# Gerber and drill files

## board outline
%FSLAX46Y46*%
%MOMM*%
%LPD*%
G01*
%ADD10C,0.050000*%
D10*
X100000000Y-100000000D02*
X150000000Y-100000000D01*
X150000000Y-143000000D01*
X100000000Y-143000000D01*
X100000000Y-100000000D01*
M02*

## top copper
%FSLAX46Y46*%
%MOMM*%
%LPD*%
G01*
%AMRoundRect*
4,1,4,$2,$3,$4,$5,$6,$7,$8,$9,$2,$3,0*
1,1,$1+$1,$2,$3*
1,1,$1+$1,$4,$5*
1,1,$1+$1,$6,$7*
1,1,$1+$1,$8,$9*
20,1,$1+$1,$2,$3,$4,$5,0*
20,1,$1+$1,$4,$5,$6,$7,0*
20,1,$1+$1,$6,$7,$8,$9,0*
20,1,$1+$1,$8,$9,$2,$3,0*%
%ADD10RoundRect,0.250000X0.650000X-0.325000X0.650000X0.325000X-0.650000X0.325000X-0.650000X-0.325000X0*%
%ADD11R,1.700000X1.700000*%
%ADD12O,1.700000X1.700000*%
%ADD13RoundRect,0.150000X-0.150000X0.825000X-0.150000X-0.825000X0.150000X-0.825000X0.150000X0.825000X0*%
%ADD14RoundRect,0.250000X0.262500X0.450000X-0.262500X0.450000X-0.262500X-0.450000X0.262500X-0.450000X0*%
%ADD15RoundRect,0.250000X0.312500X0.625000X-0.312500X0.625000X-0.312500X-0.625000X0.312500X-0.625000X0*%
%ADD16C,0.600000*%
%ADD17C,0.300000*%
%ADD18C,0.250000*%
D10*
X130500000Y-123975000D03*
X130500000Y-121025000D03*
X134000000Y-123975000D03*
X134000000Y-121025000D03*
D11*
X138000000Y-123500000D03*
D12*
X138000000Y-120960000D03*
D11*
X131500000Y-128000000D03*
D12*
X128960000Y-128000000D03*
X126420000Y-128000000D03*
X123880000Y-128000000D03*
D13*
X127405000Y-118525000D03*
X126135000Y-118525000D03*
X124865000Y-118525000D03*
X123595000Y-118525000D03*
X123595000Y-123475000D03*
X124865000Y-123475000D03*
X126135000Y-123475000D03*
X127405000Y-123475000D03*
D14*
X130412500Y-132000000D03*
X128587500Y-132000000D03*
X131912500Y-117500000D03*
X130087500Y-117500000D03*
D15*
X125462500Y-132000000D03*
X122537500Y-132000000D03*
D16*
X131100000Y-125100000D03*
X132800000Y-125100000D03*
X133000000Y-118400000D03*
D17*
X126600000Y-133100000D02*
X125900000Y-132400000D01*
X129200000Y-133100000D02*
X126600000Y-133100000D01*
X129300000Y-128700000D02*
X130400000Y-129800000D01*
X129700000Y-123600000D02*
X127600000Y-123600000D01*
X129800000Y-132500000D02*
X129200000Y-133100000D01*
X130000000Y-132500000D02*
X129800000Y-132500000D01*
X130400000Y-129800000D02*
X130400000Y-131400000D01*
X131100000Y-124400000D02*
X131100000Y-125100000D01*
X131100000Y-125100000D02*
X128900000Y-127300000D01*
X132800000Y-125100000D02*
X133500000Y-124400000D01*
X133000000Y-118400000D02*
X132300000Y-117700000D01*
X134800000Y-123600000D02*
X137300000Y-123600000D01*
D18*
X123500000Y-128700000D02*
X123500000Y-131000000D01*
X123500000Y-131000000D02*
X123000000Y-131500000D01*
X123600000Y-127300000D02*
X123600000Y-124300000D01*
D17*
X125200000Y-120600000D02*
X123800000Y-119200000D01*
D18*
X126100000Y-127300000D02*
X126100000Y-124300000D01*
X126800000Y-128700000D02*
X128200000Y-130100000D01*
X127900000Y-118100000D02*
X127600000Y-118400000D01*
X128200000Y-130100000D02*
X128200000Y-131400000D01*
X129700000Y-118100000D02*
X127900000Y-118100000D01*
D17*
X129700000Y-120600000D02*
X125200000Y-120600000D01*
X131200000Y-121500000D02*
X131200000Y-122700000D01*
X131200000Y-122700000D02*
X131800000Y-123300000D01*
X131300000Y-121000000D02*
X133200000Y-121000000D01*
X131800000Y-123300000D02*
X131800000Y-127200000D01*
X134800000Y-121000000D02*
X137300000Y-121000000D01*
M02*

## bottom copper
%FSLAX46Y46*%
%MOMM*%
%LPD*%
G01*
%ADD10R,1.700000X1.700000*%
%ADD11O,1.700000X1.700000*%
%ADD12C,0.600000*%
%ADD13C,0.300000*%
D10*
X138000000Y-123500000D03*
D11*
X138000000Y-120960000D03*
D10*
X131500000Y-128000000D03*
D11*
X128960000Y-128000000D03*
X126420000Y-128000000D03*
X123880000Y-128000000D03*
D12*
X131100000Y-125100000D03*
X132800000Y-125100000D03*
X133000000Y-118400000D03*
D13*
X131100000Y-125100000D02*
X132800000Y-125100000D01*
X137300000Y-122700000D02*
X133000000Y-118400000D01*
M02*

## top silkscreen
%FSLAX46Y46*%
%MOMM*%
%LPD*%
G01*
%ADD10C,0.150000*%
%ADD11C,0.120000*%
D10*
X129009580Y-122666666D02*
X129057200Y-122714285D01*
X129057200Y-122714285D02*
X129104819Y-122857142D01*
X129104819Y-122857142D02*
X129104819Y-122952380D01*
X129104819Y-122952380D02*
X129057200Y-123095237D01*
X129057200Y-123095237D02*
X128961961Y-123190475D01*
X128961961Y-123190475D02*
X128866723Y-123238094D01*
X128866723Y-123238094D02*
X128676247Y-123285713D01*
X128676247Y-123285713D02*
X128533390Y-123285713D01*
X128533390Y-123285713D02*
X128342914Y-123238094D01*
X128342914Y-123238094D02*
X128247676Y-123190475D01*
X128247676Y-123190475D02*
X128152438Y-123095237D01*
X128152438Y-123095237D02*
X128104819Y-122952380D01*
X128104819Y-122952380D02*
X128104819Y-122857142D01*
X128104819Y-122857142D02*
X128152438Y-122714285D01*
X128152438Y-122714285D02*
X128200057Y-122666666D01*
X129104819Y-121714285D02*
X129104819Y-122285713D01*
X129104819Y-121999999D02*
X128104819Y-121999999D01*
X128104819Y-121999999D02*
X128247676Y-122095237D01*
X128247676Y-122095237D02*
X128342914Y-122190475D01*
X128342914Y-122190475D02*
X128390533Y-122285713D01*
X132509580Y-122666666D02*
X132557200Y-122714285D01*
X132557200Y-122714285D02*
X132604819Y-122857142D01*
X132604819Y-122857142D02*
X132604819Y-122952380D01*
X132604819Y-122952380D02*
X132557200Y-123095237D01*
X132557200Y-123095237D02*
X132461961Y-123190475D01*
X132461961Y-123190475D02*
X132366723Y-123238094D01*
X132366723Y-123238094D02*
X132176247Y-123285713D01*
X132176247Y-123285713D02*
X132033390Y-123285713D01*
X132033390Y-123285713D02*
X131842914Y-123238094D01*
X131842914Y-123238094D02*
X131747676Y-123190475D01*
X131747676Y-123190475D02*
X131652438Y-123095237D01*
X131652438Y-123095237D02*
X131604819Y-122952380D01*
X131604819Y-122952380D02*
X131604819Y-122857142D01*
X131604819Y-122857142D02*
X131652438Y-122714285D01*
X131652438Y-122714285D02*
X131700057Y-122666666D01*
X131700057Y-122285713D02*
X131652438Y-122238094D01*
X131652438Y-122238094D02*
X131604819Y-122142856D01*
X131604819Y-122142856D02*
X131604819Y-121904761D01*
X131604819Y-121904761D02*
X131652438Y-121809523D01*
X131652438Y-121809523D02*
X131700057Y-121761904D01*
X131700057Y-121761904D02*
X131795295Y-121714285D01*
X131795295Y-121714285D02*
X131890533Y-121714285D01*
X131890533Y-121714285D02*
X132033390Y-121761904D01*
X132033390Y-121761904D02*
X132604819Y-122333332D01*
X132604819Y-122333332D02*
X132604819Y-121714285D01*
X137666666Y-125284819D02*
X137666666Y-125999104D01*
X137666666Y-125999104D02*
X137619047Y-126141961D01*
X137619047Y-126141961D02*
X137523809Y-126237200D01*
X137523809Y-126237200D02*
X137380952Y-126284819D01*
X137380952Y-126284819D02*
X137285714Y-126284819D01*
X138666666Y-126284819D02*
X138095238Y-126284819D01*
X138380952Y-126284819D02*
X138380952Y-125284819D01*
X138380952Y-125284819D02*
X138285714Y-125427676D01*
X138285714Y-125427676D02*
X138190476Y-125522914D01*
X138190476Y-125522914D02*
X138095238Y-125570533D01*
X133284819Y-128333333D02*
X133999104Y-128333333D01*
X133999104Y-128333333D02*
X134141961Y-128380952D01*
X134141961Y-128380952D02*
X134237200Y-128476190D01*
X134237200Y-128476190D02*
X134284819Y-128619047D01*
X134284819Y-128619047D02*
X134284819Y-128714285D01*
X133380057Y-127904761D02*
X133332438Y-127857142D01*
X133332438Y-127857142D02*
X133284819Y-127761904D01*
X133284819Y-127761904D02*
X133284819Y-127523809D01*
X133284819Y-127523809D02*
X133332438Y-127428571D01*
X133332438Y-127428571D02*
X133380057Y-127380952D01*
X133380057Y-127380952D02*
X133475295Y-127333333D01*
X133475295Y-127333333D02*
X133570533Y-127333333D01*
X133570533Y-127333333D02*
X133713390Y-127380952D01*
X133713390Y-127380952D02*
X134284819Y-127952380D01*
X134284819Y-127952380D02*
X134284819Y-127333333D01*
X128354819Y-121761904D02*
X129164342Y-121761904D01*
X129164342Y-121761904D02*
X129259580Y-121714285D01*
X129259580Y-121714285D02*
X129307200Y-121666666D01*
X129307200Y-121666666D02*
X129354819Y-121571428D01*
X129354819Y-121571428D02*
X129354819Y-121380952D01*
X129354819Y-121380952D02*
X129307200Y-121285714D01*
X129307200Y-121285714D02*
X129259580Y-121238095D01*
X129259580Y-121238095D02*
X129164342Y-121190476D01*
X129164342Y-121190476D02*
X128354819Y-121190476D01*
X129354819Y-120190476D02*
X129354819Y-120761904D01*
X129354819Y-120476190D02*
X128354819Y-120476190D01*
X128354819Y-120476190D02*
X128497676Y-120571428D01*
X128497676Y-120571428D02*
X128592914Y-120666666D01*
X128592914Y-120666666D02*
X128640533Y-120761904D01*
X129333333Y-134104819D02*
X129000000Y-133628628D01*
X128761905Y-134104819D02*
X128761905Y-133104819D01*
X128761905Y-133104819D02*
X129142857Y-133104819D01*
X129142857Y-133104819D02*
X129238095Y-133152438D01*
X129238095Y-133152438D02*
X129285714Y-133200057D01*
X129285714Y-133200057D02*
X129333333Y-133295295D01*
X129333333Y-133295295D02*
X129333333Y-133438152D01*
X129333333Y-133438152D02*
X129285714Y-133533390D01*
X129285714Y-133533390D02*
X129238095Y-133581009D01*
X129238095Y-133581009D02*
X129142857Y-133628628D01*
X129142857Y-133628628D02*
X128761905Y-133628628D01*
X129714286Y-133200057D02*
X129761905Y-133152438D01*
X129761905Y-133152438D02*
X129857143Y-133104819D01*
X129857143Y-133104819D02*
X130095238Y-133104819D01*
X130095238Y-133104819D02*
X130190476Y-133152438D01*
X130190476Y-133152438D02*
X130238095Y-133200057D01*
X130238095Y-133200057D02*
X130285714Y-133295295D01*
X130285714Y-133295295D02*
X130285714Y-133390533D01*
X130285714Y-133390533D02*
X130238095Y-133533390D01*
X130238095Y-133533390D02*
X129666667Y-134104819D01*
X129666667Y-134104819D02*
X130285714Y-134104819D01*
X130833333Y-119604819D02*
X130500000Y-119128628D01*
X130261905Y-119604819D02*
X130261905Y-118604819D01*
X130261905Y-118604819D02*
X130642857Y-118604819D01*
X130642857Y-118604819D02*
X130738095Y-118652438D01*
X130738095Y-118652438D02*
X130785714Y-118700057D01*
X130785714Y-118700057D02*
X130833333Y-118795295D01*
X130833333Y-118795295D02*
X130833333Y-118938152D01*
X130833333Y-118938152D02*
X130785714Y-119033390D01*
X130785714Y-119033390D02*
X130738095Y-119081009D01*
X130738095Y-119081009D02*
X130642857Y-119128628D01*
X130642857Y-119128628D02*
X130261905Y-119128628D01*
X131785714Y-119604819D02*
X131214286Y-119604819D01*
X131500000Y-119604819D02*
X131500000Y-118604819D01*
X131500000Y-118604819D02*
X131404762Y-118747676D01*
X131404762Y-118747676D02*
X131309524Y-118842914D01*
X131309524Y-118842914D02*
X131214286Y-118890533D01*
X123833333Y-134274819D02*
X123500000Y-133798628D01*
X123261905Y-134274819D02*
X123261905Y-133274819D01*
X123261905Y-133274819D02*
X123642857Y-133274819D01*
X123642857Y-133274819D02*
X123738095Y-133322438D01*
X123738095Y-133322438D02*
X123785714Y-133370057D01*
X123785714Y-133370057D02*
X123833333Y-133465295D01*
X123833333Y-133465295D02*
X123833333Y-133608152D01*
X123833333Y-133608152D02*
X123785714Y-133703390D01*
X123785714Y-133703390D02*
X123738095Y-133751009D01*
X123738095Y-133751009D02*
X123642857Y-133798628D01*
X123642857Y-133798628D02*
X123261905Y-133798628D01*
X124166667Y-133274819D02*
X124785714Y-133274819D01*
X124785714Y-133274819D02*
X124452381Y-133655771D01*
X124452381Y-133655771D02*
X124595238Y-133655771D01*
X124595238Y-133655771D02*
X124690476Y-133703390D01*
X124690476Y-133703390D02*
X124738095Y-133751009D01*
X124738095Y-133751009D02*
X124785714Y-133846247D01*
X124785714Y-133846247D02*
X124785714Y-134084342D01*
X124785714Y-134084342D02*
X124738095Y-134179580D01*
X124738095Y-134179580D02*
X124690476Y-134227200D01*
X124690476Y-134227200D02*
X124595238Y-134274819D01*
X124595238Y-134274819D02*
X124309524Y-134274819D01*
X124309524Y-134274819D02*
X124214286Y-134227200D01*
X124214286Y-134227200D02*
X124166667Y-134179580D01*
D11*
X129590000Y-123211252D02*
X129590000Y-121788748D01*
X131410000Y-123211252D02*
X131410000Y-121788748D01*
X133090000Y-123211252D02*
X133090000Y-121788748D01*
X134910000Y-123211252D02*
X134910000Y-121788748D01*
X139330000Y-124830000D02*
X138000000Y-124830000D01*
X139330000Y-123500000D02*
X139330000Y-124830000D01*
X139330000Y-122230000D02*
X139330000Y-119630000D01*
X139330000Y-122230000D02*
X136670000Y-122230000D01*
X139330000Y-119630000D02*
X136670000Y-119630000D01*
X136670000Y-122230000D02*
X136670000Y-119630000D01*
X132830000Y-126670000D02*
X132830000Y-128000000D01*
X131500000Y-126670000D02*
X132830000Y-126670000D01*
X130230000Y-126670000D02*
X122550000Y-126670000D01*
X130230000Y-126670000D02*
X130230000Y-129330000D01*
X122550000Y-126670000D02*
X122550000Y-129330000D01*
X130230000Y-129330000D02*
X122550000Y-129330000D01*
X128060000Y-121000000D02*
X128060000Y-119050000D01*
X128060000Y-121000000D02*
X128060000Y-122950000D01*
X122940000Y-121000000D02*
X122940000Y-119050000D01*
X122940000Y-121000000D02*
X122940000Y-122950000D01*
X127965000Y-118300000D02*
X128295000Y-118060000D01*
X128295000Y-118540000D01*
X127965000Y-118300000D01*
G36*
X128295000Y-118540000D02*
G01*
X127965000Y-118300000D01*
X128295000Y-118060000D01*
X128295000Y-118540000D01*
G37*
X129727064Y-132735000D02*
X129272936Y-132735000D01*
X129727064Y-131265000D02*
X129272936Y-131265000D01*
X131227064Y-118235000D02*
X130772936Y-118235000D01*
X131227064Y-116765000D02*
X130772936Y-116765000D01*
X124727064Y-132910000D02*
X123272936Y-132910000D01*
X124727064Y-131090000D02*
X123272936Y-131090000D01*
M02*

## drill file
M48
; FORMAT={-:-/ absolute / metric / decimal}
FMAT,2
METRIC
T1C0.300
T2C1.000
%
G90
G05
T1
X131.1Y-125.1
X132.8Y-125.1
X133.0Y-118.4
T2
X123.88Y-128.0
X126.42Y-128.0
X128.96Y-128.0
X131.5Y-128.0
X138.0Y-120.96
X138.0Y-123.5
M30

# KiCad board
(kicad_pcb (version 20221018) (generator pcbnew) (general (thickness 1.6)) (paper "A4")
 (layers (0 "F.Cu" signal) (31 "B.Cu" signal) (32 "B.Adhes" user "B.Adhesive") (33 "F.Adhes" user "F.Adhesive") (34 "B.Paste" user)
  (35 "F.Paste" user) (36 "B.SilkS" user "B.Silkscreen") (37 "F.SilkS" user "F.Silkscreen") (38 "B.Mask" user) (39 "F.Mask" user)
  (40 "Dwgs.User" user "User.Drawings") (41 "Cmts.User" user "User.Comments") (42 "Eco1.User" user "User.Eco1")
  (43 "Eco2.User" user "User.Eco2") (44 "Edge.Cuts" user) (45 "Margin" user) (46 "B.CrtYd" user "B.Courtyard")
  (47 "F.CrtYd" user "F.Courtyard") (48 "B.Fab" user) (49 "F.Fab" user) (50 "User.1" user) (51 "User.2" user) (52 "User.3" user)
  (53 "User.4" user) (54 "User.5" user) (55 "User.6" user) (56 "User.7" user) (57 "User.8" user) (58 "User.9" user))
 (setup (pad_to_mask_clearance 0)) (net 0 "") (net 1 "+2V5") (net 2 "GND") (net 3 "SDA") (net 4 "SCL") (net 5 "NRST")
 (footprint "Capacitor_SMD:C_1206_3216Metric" (layer "F.Cu") (at 130.5 122.5 90)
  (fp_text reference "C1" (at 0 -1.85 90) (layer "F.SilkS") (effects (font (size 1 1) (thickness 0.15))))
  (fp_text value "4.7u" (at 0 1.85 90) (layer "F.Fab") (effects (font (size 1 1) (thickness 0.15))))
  (fp_line (start -0.711252 -0.91) (end 0.711252 -0.91) (stroke (width 0.12) (type solid)) (layer "F.SilkS"))
  (fp_line (start -0.711252 0.91) (end 0.711252 0.91) (stroke (width 0.12) (type solid)) (layer "F.SilkS"))
  (pad "1" smd roundrect (at -1.475 0 90) (size 1.15 1.8) (layers "F.Cu" "F.Paste" "F.Mask") (roundrect_rratio 0.217391) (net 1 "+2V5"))
  (pad "2" smd roundrect (at 1.475 0 90) (size 1.15 1.8) (layers "F.Cu" "F.Paste" "F.Mask") (roundrect_rratio 0.217391) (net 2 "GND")))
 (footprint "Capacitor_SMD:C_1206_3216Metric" (layer "F.Cu") (at 134 122.5 90)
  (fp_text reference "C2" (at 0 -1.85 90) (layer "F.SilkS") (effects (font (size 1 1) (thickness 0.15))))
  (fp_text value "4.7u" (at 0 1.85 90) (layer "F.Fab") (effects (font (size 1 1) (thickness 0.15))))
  (fp_line (start -0.711252 -0.91) (end 0.711252 -0.91) (stroke (width 0.12) (type solid)) (layer "F.SilkS"))
  (fp_line (start -0.711252 0.91) (end 0.711252 0.91) (stroke (width 0.12) (type solid)) (layer "F.SilkS"))
  (pad "1" smd roundrect (at -1.475 0 90) (size 1.15 1.8) (layers "F.Cu" "F.Paste" "F.Mask") (roundrect_rratio 0.217391) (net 1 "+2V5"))
  (pad "2" smd roundrect (at 1.475 0 90) (size 1.15 1.8) (layers "F.Cu" "F.Paste" "F.Mask") (roundrect_rratio 0.217391) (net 2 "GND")))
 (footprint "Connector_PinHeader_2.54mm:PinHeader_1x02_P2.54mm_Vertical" (layer "F.Cu") (at 138 123.5 180)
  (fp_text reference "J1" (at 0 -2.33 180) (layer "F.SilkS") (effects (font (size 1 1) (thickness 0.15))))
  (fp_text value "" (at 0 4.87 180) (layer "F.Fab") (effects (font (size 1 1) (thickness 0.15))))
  (fp_line (start -1.33 -1.33) (end 0 -1.33) (stroke (width 0.12) (type solid)) (layer "F.SilkS"))
  (fp_line (start -1.33 0) (end -1.33 -1.33) (stroke (width 0.12) (type solid)) (layer "F.SilkS"))
  (fp_line (start -1.33 1.27) (end -1.33 3.87) (stroke (width 0.12) (type solid)) (layer "F.SilkS"))
  (fp_line (start -1.33 1.27) (end 1.33 1.27) (stroke (width 0.12) (type solid)) (layer "F.SilkS"))
  (fp_line (start -1.33 3.87) (end 1.33 3.87) (stroke (width 0.12) (type solid)) (layer "F.SilkS"))
  (fp_line (start 1.33 1.27) (end 1.33 3.87) (stroke (width 0.12) (type solid)) (layer "F.SilkS"))
  (pad "1" thru_hole rect (at 0 0 180) (size 1.7 1.7) (drill 1) (layers "*.Cu" "*.Mask") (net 1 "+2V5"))
  (pad "2" thru_hole oval (at 0 2.54 180) (size 1.7 1.7) (drill 1) (layers "*.Cu" "*.Mask") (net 2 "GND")))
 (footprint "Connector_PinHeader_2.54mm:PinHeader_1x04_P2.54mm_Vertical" (layer "F.Cu") (at 131.5 128 -90)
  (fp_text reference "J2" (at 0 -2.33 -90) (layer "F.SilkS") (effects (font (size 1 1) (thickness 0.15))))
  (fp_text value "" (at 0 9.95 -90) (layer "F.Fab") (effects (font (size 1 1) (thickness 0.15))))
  (fp_line (start -1.33 -1.33) (end 0 -1.33) (stroke (width 0.12) (type solid)) (layer "F.SilkS"))
  (fp_line (start -1.33 0) (end -1.33 -1.33) (stroke (width 0.12) (type solid)) (layer "F.SilkS"))
  (fp_line (start -1.33 1.27) (end -1.33 8.95) (stroke (width 0.12) (type solid)) (layer "F.SilkS"))
  (fp_line (start -1.33 1.27) (end 1.33 1.27) (stroke (width 0.12) (type solid)) (layer "F.SilkS"))
  (fp_line (start -1.33 8.95) (end 1.33 8.95) (stroke (width 0.12) (type solid)) (layer "F.SilkS"))
  (fp_line (start 1.33 1.27) (end 1.33 8.95) (stroke (width 0.12) (type solid)) (layer "F.SilkS"))
  (pad "1" thru_hole rect (at 0 0 270) (size 1.7 1.7) (drill 1) (layers "*.Cu" "*.Mask") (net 2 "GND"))
  (pad "2" thru_hole oval (at 0 2.54 270) (size 1.7 1.7) (drill 1) (layers "*.Cu" "*.Mask") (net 1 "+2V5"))
  (pad "3" thru_hole oval (at 0 5.08 270) (size 1.7 1.7) (drill 1) (layers "*.Cu" "*.Mask") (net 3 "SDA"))
  (pad "4" thru_hole oval (at 0 7.62 270) (size 1.7 1.7) (drill 1) (layers "*.Cu" "*.Mask") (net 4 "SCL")))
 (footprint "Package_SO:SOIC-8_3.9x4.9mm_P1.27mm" (layer "F.Cu") (at 125.5 121 -90)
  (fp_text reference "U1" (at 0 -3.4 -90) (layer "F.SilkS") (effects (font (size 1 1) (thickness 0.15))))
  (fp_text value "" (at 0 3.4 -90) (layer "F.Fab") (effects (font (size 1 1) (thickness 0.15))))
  (fp_line (start 0 -2.56) (end -1.95 -2.56) (stroke (width 0.12) (type solid)) (layer "F.SilkS"))
  (fp_line (start 0 -2.56) (end 1.95 -2.56) (stroke (width 0.12) (type solid)) (layer "F.SilkS"))
  (fp_line (start 0 2.56) (end -1.95 2.56) (stroke (width 0.12) (type solid)) (layer "F.SilkS"))
  (fp_line (start 0 2.56) (end 1.95 2.56) (stroke (width 0.12) (type solid)) (layer "F.SilkS"))
  (fp_poly
   (pts (xy -2.7 -2.465) (xy -2.94 -2.795) (xy -2.46 -2.795) (xy -2.7 -2.465)) (stroke (width 0.12) (type solid)) (fill solid)
   (layer "F.SilkS"))
  (pad "1" smd roundrect (at -2.475 -1.905 270) (size 1.95 0.6) (layers "F.Cu" "F.Paste" "F.Mask") (roundrect_rratio 0.25) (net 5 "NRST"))
  (pad "2" smd roundrect (at -2.475 -0.635 270) (size 1.95 0.6) (layers "F.Cu" "F.Paste" "F.Mask") (roundrect_rratio 0.25))
  (pad "3" smd roundrect (at -2.475 0.635 270) (size 1.95 0.6) (layers "F.Cu" "F.Paste" "F.Mask") (roundrect_rratio 0.25))
  (pad "4" smd roundrect (at -2.475 1.905 270) (size 1.95 0.6) (layers "F.Cu" "F.Paste" "F.Mask") (roundrect_rratio 0.25) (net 2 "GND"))
  (pad "5" smd roundrect (at 2.475 1.905 270) (size 1.95 0.6) (layers "F.Cu" "F.Paste" "F.Mask") (roundrect_rratio 0.25) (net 4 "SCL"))
  (pad "6" smd roundrect (at 2.475 0.635 270) (size 1.95 0.6) (layers "F.Cu" "F.Paste" "F.Mask") (roundrect_rratio 0.25))
  (pad "7" smd roundrect (at 2.475 -0.635 270) (size 1.95 0.6) (layers "F.Cu" "F.Paste" "F.Mask") (roundrect_rratio 0.25) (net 3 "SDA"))
  (pad "8" smd roundrect (at 2.475 -1.905 270) (size 1.95 0.6) (layers "F.Cu" "F.Paste" "F.Mask") (roundrect_rratio 0.25) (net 1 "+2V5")))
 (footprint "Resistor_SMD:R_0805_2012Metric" (layer "F.Cu") (at 129.5 132 180)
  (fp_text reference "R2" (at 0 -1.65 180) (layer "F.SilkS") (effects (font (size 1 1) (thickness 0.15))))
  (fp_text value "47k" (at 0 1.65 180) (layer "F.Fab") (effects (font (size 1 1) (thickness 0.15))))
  (fp_line (start -0.227064 -0.735) (end 0.227064 -0.735) (stroke (width 0.12) (type solid)) (layer "F.SilkS"))
  (fp_line (start -0.227064 0.735) (end 0.227064 0.735) (stroke (width 0.12) (type solid)) (layer "F.SilkS"))
  (pad "1" smd roundrect (at -0.9125 0 180) (size 1.025 1.4) (layers "F.Cu" "F.Paste" "F.Mask") (roundrect_rratio 0.243902) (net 1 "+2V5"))
  (pad "2" smd roundrect (at 0.9125 0 180) (size 1.025 1.4) (layers "F.Cu" "F.Paste" "F.Mask") (roundrect_rratio 0.243902) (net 3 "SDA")))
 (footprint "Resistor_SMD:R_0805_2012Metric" (layer "F.Cu") (at 131 117.5 180)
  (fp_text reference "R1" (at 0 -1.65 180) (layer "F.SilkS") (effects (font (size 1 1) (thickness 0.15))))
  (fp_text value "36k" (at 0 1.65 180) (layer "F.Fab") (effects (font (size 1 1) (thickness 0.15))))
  (fp_line (start -0.227064 -0.735) (end 0.227064 -0.735) (stroke (width 0.12) (type solid)) (layer "F.SilkS"))
  (fp_line (start -0.227064 0.735) (end 0.227064 0.735) (stroke (width 0.12) (type solid)) (layer "F.SilkS"))
  (pad "1" smd roundrect (at -0.9125 0 180) (size 1.025 1.4) (layers "F.Cu" "F.Paste" "F.Mask") (roundrect_rratio 0.243902) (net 1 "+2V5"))
  (pad "2" smd roundrect (at 0.9125 0 180) (size 1.025 1.4) (layers "F.Cu" "F.Paste" "F.Mask") (roundrect_rratio 0.243902) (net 5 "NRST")))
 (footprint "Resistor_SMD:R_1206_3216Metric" (layer "F.Cu") (at 124 132 180)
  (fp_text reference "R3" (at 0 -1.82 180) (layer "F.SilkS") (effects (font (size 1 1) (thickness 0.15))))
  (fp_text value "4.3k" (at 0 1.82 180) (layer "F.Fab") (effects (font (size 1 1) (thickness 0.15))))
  (fp_line (start -0.727064 -0.91) (end 0.727064 -0.91) (stroke (width 0.12) (type solid)) (layer "F.SilkS"))
  (fp_line (start -0.727064 0.91) (end 0.727064 0.91) (stroke (width 0.12) (type solid)) (layer "F.SilkS"))
  (pad "1" smd roundrect (at -1.4625 0 180) (size 1.125 1.75) (layers "F.Cu" "F.Paste" "F.Mask") (roundrect_rratio 0.222222) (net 1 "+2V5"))
  (pad "2" smd roundrect (at 1.4625 0 180) (size 1.125 1.75) (layers "F.Cu" "F.Paste" "F.Mask") (roundrect_rratio 0.222222) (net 4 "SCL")))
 (gr_rect (start 100 100) (end 150 143) (stroke (width 0.05) (type default)) (fill none) (layer "Edge.Cuts"))
 (segment (start 126.6 133.1) (end 125.9 132.4) (width 0.3) (layer "F.Cu") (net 1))
 (segment (start 129.2 133.1) (end 126.6 133.1) (width 0.3) (layer "F.Cu") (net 1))
 (segment (start 129.3 128.7) (end 130.4 129.8) (width 0.3) (layer "F.Cu") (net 1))
 (segment (start 129.7 123.6) (end 127.6 123.6) (width 0.3) (layer "F.Cu") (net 1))
 (segment (start 129.8 132.5) (end 129.2 133.1) (width 0.3) (layer "F.Cu") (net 1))
 (segment (start 130 132.5) (end 129.8 132.5) (width 0.3) (layer "F.Cu") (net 1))
 (segment (start 130.4 129.8) (end 130.4 131.4) (width 0.3) (layer "F.Cu") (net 1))
 (segment (start 131.1 124.4) (end 131.1 125.1) (width 0.3) (layer "F.Cu") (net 1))
 (segment (start 131.1 125.1) (end 128.9 127.3) (width 0.3) (layer "F.Cu") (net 1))
 (segment (start 132.8 125.1) (end 133.5 124.4) (width 0.3) (layer "F.Cu") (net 1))
 (segment (start 133 118.4) (end 132.3 117.7) (width 0.3) (layer "F.Cu") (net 1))
 (segment (start 134.8 123.6) (end 137.3 123.6) (width 0.3) (layer "F.Cu") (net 1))
 (via (at 131.1 125.1) (size 0.6) (drill 0.3) (layers "F.Cu" "B.Cu") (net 1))
 (via (at 132.8 125.1) (size 0.6) (drill 0.3) (layers "F.Cu" "B.Cu") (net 1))
 (via (at 133 118.4) (size 0.6) (drill 0.3) (layers "F.Cu" "B.Cu") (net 1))
 (segment (start 123.5 128.7) (end 123.5 131) (width 0.25) (layer "F.Cu") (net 4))
 (segment (start 123.5 131) (end 123 131.5) (width 0.25) (layer "F.Cu") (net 4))
 (segment (start 123.6 127.3) (end 123.6 124.3) (width 0.25) (layer "F.Cu") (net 4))
 (segment (start 125.2 120.6) (end 123.8 119.2) (width 0.3) (layer "F.Cu") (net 2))
 (segment (start 126.1 127.3) (end 126.1 124.3) (width 0.25) (layer "F.Cu") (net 3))
 (segment (start 126.8 128.7) (end 128.2 130.1) (width 0.25) (layer "F.Cu") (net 3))
 (segment (start 127.9 118.1) (end 127.6 118.4) (width 0.25) (layer "F.Cu") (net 5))
 (segment (start 128.2 130.1) (end 128.2 131.4) (width 0.25) (layer "F.Cu") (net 3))
 (segment (start 129.7 118.1) (end 127.9 118.1) (width 0.25) (layer "F.Cu") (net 5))
 (segment (start 129.7 120.6) (end 125.2 120.6) (width 0.3) (layer "F.Cu") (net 2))
 (segment (start 131.1 125.1) (end 132.8 125.1) (width 0.3) (layer "B.Cu") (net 1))
 (segment (start 131.2 121.5) (end 131.2 122.7) (width 0.3) (layer "F.Cu") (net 2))
 (segment (start 131.2 122.7) (end 131.8 123.3) (width 0.3) (layer "F.Cu") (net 2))
 (segment (start 131.3 121) (end 133.2 121) (width 0.3) (layer "F.Cu") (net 2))
 (segment (start 131.8 123.3) (end 131.8 127.2) (width 0.3) (layer "F.Cu") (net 2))
 (segment (start 134.8 121) (end 137.3 121) (width 0.3) (layer "F.Cu") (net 2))
 (segment (start 137.3 122.7) (end 133 118.4) (width 0.3) (layer "B.Cu") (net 1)))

